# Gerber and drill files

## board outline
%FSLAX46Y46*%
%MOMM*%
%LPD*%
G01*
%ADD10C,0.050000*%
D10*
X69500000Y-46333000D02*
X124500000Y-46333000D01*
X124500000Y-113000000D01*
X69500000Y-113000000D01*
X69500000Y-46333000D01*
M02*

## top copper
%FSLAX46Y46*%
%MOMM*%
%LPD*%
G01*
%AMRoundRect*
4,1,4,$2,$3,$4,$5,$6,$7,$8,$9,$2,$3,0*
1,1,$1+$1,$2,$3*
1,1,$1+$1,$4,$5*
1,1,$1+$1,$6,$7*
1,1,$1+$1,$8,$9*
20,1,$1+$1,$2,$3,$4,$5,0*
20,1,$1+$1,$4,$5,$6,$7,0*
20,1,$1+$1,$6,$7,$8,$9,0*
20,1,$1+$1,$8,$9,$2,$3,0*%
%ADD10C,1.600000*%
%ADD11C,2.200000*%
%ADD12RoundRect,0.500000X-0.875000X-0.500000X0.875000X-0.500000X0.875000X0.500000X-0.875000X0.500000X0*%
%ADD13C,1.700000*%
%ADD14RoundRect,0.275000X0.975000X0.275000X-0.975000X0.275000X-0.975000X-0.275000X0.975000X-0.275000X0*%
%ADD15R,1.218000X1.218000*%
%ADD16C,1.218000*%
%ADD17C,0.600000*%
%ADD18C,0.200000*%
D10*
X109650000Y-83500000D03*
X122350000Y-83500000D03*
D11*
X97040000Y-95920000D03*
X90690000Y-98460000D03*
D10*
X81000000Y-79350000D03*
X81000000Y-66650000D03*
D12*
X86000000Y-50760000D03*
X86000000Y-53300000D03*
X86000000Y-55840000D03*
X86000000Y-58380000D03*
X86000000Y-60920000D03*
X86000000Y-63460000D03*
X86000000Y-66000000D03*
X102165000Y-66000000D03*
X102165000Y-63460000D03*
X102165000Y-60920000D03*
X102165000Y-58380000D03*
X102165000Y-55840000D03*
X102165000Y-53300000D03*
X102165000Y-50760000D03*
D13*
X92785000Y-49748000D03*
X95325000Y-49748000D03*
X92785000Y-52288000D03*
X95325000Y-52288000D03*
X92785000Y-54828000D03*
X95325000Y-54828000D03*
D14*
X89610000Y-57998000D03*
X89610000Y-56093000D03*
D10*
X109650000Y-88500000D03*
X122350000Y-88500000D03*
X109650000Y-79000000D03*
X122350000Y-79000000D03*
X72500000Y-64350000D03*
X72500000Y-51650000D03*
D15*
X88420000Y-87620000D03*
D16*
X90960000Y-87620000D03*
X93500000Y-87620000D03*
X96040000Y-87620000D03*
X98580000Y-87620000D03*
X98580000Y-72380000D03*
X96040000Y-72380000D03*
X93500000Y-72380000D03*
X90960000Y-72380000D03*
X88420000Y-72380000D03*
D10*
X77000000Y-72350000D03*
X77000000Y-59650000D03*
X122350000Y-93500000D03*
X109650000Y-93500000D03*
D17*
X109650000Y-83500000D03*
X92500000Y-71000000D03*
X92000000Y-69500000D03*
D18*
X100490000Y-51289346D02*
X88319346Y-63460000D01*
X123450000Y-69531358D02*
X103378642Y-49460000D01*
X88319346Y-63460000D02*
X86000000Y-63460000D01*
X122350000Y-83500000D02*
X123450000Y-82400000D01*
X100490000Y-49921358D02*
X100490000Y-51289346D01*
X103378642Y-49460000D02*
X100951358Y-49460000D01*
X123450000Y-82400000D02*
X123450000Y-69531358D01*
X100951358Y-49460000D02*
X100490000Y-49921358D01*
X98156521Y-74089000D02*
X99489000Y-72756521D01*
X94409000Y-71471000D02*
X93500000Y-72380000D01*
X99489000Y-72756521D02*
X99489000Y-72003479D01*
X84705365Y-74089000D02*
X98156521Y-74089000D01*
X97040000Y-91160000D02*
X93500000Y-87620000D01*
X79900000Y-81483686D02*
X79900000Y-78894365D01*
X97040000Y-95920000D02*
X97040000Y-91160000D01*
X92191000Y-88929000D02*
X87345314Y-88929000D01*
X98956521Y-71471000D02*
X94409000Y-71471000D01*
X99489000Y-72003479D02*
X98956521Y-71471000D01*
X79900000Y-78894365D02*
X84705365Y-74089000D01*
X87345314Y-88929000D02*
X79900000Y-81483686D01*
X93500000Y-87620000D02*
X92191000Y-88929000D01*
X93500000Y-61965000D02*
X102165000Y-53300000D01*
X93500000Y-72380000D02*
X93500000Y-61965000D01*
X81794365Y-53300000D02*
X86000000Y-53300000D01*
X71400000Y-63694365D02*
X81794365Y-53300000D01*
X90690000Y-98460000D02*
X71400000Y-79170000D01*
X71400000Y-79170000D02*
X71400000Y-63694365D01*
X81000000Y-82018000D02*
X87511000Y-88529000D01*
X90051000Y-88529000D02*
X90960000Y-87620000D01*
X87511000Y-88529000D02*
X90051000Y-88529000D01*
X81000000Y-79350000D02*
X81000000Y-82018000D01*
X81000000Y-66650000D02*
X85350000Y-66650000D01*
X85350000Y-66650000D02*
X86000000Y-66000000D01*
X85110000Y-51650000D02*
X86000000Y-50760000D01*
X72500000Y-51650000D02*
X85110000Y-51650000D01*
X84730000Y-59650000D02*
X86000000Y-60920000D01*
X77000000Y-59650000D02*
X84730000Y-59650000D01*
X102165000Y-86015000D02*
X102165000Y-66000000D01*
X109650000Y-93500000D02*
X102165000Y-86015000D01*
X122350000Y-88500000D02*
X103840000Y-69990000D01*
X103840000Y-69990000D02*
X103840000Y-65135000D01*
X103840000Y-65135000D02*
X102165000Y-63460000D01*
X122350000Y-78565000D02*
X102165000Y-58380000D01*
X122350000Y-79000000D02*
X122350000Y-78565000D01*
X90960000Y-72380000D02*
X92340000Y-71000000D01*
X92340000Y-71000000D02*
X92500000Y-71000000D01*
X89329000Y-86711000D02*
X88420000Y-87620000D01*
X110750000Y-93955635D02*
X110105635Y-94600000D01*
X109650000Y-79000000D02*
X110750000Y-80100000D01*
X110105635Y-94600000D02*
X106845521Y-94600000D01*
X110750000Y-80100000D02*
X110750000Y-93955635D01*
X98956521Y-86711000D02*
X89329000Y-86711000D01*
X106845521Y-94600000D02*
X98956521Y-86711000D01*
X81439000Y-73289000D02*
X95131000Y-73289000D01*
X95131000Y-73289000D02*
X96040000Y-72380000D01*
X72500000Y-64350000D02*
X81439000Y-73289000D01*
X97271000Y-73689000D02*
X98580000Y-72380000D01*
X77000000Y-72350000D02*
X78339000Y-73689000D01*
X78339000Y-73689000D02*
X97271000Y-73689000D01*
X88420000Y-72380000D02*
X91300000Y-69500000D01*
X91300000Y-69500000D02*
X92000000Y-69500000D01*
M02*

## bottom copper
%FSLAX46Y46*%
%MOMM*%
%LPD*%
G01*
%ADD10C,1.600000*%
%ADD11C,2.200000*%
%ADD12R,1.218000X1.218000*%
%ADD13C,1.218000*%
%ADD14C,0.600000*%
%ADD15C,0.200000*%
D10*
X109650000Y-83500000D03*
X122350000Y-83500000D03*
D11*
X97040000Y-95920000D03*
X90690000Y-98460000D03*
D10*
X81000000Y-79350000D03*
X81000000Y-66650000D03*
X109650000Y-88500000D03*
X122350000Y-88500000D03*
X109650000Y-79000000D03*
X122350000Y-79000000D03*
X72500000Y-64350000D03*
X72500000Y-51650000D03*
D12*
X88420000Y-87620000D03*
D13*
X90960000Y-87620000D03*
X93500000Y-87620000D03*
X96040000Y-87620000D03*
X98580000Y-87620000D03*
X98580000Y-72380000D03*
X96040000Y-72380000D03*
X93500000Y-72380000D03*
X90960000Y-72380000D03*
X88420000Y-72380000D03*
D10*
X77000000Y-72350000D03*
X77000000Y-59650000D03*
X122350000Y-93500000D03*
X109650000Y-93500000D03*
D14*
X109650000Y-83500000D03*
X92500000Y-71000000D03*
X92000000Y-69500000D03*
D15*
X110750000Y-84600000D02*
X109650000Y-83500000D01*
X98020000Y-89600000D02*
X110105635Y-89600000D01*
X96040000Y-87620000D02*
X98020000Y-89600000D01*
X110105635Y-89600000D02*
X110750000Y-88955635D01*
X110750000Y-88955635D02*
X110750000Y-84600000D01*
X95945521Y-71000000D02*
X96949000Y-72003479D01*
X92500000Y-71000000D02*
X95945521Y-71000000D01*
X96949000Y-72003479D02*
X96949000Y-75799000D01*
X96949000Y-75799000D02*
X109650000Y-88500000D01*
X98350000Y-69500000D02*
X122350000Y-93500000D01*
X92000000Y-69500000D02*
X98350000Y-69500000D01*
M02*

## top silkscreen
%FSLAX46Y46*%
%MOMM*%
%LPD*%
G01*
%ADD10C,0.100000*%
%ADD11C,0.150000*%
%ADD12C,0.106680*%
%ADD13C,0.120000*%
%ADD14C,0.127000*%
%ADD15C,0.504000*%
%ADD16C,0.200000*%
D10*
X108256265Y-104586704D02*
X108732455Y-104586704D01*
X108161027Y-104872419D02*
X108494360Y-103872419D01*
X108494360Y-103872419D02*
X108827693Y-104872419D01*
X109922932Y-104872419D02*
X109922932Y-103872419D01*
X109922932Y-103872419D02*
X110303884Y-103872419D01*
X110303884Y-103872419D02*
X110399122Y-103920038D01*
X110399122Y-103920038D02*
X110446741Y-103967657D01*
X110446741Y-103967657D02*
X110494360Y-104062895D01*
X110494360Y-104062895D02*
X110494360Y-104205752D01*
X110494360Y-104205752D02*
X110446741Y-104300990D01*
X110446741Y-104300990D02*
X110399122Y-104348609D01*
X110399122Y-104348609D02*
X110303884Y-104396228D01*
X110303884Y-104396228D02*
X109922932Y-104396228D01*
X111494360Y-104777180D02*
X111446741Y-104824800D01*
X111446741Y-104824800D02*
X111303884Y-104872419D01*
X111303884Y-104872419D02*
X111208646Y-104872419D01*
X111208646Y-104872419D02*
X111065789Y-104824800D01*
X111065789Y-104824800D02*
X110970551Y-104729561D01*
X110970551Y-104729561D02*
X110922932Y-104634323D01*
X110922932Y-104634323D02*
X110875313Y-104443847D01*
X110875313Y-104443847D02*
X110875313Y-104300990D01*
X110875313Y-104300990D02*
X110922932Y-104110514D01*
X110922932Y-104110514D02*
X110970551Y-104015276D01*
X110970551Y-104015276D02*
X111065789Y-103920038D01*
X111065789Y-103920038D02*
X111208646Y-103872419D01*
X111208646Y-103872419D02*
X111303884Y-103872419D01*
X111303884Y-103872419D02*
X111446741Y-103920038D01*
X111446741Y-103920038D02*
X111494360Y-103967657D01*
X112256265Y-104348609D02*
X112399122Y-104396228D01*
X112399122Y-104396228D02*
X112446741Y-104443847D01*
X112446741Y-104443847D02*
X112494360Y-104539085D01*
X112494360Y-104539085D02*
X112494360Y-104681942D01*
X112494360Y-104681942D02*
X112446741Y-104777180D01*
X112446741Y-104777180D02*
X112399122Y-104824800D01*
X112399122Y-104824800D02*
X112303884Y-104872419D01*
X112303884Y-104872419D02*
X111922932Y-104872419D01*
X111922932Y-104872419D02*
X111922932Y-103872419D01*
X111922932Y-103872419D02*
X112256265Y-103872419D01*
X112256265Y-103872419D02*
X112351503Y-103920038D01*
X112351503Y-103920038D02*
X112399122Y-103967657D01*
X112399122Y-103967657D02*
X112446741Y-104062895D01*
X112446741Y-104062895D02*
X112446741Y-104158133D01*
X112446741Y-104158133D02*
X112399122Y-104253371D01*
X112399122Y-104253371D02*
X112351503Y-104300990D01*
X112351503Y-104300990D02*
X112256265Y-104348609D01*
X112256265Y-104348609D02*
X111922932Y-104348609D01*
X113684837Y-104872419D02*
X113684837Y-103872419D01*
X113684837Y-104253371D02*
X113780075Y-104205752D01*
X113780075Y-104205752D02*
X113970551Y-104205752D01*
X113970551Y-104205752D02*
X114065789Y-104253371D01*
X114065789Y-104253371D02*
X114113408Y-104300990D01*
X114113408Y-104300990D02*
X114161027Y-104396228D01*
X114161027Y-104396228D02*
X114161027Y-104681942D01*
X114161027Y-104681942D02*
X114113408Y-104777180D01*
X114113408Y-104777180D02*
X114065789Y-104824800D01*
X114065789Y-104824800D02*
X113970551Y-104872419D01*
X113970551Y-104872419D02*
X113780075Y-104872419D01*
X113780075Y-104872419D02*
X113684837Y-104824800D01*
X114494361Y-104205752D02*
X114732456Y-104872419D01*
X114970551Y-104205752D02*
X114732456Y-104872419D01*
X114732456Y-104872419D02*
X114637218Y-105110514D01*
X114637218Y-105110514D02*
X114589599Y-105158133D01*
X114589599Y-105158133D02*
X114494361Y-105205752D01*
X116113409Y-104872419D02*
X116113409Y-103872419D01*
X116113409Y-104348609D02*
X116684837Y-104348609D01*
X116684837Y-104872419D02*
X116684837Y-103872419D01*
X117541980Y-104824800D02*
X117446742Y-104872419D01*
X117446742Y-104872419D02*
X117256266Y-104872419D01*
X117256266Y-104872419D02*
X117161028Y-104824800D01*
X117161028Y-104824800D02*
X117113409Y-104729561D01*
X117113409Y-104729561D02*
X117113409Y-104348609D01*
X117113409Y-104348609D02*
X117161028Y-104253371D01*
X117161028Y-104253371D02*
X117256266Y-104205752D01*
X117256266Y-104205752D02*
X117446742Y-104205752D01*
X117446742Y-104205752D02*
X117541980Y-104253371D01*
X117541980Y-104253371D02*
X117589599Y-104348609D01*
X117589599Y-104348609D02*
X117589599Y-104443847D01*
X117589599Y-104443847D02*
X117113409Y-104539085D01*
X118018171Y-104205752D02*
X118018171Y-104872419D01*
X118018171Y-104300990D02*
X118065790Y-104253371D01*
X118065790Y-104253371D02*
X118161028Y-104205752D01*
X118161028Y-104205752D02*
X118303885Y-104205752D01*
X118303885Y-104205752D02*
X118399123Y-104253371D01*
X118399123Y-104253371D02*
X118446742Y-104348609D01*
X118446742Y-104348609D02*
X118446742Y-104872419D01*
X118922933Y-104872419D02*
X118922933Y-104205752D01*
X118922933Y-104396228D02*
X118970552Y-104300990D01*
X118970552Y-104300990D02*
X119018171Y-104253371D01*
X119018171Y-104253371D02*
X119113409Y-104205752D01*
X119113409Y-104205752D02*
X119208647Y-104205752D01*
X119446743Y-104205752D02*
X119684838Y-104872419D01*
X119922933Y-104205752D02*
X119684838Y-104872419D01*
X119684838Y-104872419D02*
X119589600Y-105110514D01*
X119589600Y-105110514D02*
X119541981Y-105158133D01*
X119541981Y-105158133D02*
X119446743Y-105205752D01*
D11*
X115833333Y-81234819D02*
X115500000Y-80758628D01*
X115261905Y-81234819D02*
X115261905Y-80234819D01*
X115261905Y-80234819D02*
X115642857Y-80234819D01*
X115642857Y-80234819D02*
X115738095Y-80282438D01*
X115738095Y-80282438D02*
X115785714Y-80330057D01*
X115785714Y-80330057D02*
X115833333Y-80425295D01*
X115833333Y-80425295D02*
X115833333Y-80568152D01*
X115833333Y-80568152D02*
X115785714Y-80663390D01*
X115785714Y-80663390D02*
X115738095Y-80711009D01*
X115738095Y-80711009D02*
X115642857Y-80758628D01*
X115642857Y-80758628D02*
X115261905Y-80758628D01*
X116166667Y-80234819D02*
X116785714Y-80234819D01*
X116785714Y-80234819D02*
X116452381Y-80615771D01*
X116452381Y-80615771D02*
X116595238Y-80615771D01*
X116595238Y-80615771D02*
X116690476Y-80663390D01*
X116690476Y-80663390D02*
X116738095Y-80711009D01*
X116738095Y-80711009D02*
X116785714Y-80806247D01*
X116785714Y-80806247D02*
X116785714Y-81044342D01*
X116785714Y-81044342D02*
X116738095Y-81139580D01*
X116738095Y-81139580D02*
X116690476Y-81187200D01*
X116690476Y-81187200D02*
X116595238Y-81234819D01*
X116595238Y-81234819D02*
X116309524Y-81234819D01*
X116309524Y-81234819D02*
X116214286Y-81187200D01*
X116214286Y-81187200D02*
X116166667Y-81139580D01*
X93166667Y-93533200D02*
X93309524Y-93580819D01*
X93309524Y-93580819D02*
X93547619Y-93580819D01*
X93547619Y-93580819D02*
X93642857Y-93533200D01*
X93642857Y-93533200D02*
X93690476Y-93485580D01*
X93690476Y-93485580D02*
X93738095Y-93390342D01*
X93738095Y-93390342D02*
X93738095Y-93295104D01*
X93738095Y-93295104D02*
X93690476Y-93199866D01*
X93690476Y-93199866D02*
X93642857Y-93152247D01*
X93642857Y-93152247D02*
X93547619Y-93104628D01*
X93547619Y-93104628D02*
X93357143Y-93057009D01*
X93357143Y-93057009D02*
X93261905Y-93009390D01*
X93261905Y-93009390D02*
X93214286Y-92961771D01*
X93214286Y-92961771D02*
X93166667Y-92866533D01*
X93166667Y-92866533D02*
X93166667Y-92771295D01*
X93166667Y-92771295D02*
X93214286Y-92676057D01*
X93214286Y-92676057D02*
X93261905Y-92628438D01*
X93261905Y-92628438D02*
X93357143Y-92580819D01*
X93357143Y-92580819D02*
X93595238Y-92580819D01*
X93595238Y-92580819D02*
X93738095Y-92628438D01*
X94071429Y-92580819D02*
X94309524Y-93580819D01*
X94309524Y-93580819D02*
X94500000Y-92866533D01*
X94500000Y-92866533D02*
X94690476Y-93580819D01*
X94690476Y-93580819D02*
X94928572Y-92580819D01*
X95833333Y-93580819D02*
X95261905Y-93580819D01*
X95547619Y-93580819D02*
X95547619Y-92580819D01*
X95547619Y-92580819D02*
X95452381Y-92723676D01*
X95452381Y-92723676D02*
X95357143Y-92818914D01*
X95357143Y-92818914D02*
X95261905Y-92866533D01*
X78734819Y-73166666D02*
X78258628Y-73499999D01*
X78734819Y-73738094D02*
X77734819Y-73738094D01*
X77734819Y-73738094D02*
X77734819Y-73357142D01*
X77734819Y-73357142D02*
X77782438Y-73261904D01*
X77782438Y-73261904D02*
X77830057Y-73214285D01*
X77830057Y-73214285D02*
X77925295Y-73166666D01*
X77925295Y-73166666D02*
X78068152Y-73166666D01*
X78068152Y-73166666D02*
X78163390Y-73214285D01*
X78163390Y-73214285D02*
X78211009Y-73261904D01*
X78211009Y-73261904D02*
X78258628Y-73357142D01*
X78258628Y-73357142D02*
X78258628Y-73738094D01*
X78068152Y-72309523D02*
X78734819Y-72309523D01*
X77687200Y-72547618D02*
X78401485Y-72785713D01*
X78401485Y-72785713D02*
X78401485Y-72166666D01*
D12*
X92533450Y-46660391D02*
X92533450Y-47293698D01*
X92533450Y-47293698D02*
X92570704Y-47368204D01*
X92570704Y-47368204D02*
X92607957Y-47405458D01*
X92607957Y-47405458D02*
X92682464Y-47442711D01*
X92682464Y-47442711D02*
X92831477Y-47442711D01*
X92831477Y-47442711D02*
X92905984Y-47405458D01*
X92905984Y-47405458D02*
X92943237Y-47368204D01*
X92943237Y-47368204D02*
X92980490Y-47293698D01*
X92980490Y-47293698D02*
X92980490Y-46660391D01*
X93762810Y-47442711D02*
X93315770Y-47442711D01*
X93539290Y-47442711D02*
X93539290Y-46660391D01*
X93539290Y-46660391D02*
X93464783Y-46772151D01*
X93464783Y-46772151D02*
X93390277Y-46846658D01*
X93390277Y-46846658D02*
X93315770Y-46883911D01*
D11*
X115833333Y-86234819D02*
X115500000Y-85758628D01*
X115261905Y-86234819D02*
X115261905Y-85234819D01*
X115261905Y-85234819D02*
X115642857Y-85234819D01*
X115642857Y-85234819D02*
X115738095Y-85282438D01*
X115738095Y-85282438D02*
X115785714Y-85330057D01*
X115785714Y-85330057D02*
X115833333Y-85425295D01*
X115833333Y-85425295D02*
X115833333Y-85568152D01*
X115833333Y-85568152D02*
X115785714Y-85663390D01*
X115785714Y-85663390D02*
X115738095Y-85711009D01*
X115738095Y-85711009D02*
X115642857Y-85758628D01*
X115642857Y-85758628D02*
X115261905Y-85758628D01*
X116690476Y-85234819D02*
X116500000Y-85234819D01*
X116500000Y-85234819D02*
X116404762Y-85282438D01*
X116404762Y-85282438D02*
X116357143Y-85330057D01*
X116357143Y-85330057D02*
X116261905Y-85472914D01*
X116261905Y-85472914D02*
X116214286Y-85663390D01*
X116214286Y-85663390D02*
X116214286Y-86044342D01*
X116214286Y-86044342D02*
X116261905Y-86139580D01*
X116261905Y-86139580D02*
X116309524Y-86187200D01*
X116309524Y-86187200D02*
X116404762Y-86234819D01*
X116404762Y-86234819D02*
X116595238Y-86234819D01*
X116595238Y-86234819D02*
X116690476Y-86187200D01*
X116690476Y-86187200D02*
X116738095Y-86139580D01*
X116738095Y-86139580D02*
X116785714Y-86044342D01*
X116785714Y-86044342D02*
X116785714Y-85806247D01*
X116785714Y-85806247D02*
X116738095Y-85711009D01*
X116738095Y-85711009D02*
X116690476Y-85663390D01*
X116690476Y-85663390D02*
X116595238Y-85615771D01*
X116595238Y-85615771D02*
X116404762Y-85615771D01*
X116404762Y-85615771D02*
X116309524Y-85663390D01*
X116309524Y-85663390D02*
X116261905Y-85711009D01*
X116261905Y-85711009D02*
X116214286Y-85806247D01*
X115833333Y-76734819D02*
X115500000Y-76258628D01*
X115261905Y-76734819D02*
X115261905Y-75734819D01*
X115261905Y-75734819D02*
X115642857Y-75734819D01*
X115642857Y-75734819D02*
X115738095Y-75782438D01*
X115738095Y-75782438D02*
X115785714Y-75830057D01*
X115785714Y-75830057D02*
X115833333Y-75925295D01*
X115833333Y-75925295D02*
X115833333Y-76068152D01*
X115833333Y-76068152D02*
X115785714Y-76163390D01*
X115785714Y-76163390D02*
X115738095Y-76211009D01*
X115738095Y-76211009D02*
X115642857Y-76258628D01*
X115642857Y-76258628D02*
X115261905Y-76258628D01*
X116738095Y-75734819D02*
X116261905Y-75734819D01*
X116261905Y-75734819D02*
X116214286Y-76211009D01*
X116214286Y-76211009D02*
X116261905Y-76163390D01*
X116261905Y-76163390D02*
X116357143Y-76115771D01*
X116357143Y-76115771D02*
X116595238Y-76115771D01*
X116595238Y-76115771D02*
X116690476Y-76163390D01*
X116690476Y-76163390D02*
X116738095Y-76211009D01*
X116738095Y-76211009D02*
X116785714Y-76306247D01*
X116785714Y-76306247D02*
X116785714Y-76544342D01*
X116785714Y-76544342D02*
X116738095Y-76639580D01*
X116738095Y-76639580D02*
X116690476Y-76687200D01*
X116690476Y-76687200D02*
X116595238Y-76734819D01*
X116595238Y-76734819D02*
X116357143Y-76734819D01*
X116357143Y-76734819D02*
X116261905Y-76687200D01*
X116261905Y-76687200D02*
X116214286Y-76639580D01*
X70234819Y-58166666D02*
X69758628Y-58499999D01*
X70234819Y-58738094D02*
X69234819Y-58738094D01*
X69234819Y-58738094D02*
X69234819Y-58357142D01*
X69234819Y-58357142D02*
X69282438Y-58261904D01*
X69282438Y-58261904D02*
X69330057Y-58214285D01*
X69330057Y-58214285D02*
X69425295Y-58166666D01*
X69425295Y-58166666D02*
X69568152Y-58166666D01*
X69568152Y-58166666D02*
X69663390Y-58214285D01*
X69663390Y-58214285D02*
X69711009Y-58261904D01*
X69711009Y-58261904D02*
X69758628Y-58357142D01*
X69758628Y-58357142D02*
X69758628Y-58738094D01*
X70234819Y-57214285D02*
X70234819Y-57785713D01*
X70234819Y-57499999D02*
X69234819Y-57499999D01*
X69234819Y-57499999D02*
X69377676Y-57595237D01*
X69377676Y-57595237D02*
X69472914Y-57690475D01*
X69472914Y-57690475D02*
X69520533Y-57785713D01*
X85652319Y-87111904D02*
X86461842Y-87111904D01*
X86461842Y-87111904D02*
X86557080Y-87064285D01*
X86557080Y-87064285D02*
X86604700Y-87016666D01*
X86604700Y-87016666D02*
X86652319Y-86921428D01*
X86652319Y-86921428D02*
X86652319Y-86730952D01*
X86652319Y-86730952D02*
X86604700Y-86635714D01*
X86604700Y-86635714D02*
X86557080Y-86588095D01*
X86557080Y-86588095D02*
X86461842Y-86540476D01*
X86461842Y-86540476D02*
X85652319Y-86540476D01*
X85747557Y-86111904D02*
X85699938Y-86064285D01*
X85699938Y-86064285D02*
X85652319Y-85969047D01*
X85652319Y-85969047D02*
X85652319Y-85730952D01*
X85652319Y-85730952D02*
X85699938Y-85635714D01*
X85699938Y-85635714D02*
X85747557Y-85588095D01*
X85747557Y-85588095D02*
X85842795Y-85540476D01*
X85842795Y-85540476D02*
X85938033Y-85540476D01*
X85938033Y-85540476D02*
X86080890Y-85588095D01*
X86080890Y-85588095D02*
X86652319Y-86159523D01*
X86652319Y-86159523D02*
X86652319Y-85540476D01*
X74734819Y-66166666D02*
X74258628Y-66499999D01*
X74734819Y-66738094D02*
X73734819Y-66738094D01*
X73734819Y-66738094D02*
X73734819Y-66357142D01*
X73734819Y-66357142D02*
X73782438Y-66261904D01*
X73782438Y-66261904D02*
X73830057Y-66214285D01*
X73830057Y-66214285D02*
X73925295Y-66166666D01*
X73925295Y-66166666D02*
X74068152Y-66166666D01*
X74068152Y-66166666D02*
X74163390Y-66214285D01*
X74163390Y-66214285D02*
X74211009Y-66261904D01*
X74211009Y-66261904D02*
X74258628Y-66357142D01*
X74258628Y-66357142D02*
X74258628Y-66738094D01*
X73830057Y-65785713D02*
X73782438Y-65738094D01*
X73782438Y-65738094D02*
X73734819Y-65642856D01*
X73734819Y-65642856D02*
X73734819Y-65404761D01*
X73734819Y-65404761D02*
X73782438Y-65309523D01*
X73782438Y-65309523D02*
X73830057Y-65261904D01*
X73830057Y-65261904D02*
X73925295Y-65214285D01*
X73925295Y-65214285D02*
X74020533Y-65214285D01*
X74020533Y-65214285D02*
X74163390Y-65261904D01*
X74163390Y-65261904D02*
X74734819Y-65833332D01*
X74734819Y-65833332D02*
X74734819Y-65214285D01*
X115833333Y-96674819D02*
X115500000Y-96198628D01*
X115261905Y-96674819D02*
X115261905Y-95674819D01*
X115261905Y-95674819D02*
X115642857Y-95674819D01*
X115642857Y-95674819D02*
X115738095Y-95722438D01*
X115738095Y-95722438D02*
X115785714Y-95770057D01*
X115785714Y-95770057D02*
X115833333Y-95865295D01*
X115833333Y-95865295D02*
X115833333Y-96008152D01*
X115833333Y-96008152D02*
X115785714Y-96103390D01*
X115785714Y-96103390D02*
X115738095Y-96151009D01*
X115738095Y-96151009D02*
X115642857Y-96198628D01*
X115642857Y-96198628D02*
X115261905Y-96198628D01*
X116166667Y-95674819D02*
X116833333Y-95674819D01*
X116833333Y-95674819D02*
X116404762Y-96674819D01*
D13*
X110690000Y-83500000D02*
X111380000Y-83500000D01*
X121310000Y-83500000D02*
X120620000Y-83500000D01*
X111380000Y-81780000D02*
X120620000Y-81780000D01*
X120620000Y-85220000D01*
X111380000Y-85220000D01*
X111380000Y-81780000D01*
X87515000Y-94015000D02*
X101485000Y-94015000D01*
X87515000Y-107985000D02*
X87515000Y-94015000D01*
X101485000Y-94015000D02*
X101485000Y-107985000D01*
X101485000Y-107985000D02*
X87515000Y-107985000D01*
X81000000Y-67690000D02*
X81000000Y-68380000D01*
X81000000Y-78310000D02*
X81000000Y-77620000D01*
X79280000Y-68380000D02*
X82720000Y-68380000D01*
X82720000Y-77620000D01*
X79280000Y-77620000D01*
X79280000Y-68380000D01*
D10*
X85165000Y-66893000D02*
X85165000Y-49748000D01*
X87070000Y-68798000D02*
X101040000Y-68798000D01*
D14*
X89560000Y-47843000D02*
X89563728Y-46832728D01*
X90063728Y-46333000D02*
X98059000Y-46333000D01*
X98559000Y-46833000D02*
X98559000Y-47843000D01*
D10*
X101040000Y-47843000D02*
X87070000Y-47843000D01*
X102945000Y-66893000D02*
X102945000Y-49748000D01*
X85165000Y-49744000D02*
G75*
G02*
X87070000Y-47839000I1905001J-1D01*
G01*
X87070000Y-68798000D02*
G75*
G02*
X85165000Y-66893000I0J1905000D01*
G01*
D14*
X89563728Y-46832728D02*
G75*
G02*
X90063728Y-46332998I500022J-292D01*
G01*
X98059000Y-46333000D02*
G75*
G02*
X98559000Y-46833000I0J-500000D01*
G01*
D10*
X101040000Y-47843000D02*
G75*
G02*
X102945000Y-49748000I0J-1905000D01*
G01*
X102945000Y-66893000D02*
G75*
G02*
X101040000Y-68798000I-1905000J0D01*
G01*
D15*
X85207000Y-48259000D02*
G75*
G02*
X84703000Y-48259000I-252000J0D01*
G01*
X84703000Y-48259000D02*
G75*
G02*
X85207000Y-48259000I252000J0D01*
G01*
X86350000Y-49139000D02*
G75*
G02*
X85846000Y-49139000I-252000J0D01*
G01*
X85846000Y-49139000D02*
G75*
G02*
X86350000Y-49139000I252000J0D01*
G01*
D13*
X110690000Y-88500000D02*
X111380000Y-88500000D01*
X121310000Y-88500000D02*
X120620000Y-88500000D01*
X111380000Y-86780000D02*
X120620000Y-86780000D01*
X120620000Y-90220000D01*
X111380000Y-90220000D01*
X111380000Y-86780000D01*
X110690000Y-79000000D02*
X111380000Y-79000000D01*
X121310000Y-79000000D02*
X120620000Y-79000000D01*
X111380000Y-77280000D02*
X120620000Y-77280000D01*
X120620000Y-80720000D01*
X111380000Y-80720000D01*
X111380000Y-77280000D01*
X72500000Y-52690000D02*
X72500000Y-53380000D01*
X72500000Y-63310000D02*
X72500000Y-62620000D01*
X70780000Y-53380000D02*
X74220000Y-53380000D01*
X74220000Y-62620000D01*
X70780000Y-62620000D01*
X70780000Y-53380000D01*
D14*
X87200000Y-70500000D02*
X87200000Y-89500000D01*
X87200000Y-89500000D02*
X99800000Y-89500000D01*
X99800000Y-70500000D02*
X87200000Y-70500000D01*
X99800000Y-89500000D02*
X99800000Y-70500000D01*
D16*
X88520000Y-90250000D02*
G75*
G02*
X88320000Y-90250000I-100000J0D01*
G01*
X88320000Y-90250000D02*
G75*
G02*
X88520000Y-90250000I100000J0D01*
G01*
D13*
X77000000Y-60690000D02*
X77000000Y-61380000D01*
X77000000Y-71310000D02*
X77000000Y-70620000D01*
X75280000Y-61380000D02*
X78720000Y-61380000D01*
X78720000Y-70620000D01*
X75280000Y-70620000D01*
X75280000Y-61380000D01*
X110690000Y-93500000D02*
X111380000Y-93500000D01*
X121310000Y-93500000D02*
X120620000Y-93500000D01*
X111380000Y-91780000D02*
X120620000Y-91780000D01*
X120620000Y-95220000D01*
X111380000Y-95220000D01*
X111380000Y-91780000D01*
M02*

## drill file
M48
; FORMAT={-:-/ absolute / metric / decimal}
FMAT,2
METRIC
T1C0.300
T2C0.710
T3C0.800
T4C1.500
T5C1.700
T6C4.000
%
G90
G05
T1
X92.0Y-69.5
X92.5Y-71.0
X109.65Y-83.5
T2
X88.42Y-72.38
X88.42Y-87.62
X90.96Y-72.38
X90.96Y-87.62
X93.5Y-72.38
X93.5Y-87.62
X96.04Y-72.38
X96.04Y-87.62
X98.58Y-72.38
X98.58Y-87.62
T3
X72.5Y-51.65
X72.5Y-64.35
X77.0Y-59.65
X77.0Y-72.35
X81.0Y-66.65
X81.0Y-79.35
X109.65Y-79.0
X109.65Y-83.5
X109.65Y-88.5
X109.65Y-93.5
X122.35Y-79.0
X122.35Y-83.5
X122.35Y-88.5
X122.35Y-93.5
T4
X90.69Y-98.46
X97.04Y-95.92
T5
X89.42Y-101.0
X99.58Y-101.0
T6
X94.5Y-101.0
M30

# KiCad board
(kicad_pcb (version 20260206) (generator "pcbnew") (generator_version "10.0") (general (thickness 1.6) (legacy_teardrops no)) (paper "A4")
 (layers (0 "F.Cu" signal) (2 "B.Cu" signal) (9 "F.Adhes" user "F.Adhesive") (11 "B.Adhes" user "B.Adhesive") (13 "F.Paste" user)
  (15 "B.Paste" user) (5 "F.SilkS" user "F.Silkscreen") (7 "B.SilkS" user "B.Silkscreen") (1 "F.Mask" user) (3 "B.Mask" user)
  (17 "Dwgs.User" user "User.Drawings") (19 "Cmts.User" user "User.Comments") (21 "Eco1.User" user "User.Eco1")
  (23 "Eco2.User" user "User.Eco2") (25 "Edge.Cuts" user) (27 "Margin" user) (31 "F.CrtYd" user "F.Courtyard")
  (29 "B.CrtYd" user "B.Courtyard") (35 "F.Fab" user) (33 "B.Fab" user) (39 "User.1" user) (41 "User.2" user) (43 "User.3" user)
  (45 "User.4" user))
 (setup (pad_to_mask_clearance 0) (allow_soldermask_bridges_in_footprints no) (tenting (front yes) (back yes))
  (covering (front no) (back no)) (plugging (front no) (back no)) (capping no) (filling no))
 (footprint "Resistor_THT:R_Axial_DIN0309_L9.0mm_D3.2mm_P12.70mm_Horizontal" (layer "F.Cu") (at 109.65 83.5)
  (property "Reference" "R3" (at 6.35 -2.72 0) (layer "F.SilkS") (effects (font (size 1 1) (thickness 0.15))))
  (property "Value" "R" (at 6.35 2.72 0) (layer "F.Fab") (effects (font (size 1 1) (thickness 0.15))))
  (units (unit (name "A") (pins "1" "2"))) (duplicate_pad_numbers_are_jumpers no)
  (fp_line (start 1.04 0) (end 1.73 0) (stroke (width 0.12) (type solid)) (layer "F.SilkS"))
  (fp_line (start 11.66 0) (end 10.97 0) (stroke (width 0.12) (type solid)) (layer "F.SilkS"))
  (fp_rect (start 1.73 -1.72) (end 10.97 1.72) (stroke (width 0.12) (type solid)) (fill no) (layer "F.SilkS"))
  (pad "1" thru_hole circle (at 0 0) (size 1.6 1.6) (drill 0.8) (layers "*.Cu" "*.Mask") (remove_unused_layers no) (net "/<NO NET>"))
  (pad "2" thru_hole circle (at 12.7 0) (size 1.6 1.6) (drill 0.8) (layers "*.Cu" "*.Mask") (remove_unused_layers no) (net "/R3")))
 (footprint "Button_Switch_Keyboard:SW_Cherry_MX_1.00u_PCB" (layer "F.Cu") (at 97.04 95.92)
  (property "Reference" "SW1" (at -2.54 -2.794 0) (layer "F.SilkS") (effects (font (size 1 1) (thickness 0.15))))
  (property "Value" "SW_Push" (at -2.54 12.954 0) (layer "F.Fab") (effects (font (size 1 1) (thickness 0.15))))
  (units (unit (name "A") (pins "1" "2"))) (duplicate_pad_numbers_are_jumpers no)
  (fp_line (start -9.525 -1.905) (end 4.445 -1.905) (stroke (width 0.12) (type solid)) (layer "F.SilkS"))
  (fp_line (start -9.525 12.065) (end -9.525 -1.905) (stroke (width 0.12) (type solid)) (layer "F.SilkS"))
  (fp_line (start 4.445 -1.905) (end 4.445 12.065) (stroke (width 0.12) (type solid)) (layer "F.SilkS"))
  (fp_line (start 4.445 12.065) (end -9.525 12.065) (stroke (width 0.12) (type solid)) (layer "F.SilkS"))
  (pad "" np_thru_hole circle (at -7.62 5.08) (size 1.7 1.7) (drill 1.7) (layers "*.Cu" "*.Mask"))
  (pad "" np_thru_hole circle (at -2.54 5.08) (size 4 4) (drill 4) (layers "*.Cu" "*.Mask"))
  (pad "" np_thru_hole circle (at 2.54 5.08) (size 1.7 1.7) (drill 1.7) (layers "*.Cu" "*.Mask"))
  (pad "1" thru_hole circle (at 0 0) (size 2.2 2.2) (drill 1.5) (layers "*.Cu" "*.Mask") (remove_unused_layers no) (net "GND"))
  (pad "2" thru_hole circle (at -6.35 2.54) (size 2.2 2.2) (drill 1.5) (layers "*.Cu" "*.Mask") (remove_unused_layers no) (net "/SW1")))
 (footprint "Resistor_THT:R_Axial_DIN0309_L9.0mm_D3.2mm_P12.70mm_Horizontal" (layer "F.Cu") (at 81 79.35 90)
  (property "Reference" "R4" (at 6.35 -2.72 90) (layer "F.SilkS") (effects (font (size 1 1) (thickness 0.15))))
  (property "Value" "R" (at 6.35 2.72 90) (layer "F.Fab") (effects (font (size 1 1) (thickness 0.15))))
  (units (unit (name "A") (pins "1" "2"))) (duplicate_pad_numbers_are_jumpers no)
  (fp_line (start 11.66 0) (end 10.97 0) (stroke (width 0.12) (type solid)) (layer "F.SilkS"))
  (fp_line (start 1.04 0) (end 1.73 0) (stroke (width 0.12) (type solid)) (layer "F.SilkS"))
  (fp_rect (start 1.73 -1.72) (end 10.97 1.72) (stroke (width 0.12) (type solid)) (fill no) (layer "F.SilkS"))
  (pad "1" thru_hole circle (at 0 0 90) (size 1.6 1.6) (drill 0.8) (layers "*.Cu" "*.Mask") (remove_unused_layers no) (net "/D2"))
  (pad "2" thru_hole circle (at 12.7 0 90) (size 1.6 1.6) (drill 0.8) (layers "*.Cu" "*.Mask") (remove_unused_layers no) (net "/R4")))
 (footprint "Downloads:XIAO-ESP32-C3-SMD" (layer "F.Cu") (at 85.165 68.88)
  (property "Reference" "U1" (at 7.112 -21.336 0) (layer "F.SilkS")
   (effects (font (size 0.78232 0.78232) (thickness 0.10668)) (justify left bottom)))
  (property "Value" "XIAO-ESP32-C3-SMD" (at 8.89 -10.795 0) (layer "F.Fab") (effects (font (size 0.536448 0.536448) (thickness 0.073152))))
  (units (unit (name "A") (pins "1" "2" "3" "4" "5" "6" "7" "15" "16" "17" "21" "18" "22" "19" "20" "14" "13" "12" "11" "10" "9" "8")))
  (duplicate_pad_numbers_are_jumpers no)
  (fp_line (start 0 -1.987) (end 0 -19.132) (stroke (width 0.1) (type solid)) (layer "F.SilkS"))
  (fp_line (start 1.905 -0.082) (end 15.875 -0.082) (stroke (width 0.1) (type solid)) (layer "F.SilkS"))
  (fp_line (start 4.395 -21.037) (end 4.398728 -22.047272) (stroke (width 0.127) (type solid)) (layer "F.SilkS"))
  (fp_line (start 4.898728 -22.547) (end 12.894 -22.547) (stroke (width 0.127) (type solid)) (layer "F.SilkS"))
  (fp_line (start 13.394 -22.047) (end 13.394 -21.037) (stroke (width 0.127) (type solid)) (layer "F.SilkS"))
  (fp_line (start 15.875 -21.037) (end 1.905 -21.037) (stroke (width 0.1) (type solid)) (layer "F.SilkS"))
  (fp_line (start 17.78 -1.987) (end 17.78 -19.132) (stroke (width 0.1) (type solid)) (layer "F.SilkS"))
  (fp_arc (start 0 -19.136) (mid 0.557962 -20.483038) (end 1.905 -21.041) (stroke (width 0.1) (type solid)) (layer "F.SilkS"))
  (fp_arc (start 1.905 -0.082) (mid 0.557962 -0.639962) (end 0 -1.987) (stroke (width 0.1) (type solid)) (layer "F.SilkS"))
  (fp_arc (start 4.398728 -22.047272) (mid 4.545272 -22.40064) (end 4.898728 -22.547) (stroke (width 0.127) (type default))
   (layer "F.SilkS"))
  (fp_arc (start 12.894 -22.547) (mid 13.247553 -22.400553) (end 13.394 -22.047) (stroke (width 0.127) (type default)) (layer "F.SilkS"))
  (fp_arc (start 15.875 -21.037) (mid 17.222038 -20.479038) (end 17.78 -19.132) (stroke (width 0.1) (type solid)) (layer "F.SilkS"))
  (fp_arc (start 17.78 -1.987) (mid 17.222038 -0.639962) (end 15.875 -0.082) (stroke (width 0.1) (type solid)) (layer "F.SilkS"))
  (fp_circle (center -0.21 -20.621) (end -0.21 -20.875) (stroke (width 0.5) (type solid)) (fill yes) (layer "F.SilkS"))
  (fp_circle (center 0.933 -19.741) (end 0.933 -19.995) (stroke (width 0.5) (type solid)) (fill yes) (layer "F.SilkS"))
  (pad "1" smd roundrect (at 0.835 -18.12) (size 2.75 2) (layers "F.Cu" "F.Mask" "F.Paste") (roundrect_rratio 0.25) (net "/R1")
   (solder_mask_margin 0.0508) (thermal_bridge_angle 45))
  (pad "2" smd roundrect (at 0.835 -15.58) (size 2.75 2) (layers "F.Cu" "F.Mask" "F.Paste") (roundrect_rratio 0.25) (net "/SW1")
   (solder_mask_margin 0.0508) (thermal_bridge_angle 45))
  (pad "3" smd roundrect (at 0.835 -13.04) (size 2.75 2) (layers "F.Cu" "F.Mask" "F.Paste") (roundrect_rratio 0.25)
   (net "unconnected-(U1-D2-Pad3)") (solder_mask_margin 0.0508) (thermal_bridge_angle 45))
  (pad "4" smd roundrect (at 0.835 -10.5) (size 2.75 2) (layers "F.Cu" "F.Mask" "F.Paste") (roundrect_rratio 0.25)
   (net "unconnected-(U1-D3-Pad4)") (solder_mask_margin 0.0508) (thermal_bridge_angle 45))
  (pad "5" smd roundrect (at 0.835 -7.96) (size 2.75 2) (layers "F.Cu" "F.Mask" "F.Paste") (roundrect_rratio 0.25) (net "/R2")
   (solder_mask_margin 0.0508) (thermal_bridge_angle 45))
  (pad "6" smd roundrect (at 0.835 -5.42) (size 2.75 2) (layers "F.Cu" "F.Mask" "F.Paste") (roundrect_rratio 0.25) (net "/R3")
   (solder_mask_margin 0.0508) (thermal_bridge_angle 45))
  (pad "7" smd roundrect (at 0.835 -2.88) (size 2.75 2) (layers "F.Cu" "F.Mask" "F.Paste") (roundrect_rratio 0.25) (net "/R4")
   (solder_mask_margin 0.0508) (thermal_bridge_angle 45))
  (pad "8" smd roundrect (at 17 -2.88) (size 2.75 2) (layers "F.Cu" "F.Mask" "F.Paste") (roundrect_rratio 0.25) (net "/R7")
   (solder_mask_margin 0.0508) (thermal_bridge_angle 45))
  (pad "9" smd roundrect (at 17 -5.42) (size 2.75 2) (layers "F.Cu" "F.Mask" "F.Paste") (roundrect_rratio 0.25) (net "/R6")
   (solder_mask_margin 0.0508) (thermal_bridge_angle 45))
  (pad "10" smd roundrect (at 17 -7.96) (size 2.75 2) (layers "F.Cu" "F.Mask" "F.Paste") (roundrect_rratio 0.25)
   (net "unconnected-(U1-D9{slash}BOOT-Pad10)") (solder_mask_margin 0.0508) (thermal_bridge_angle 45))
  (pad "11" smd roundrect (at 17 -10.5) (size 2.75 2) (layers "F.Cu" "F.Mask" "F.Paste") (roundrect_rratio 0.25) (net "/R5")
   (solder_mask_margin 0.0508) (thermal_bridge_angle 45))
  (pad "12" smd roundrect (at 17 -13.04) (size 2.75 2) (layers "F.Cu" "F.Mask" "F.Paste") (roundrect_rratio 0.25) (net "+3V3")
   (solder_mask_margin 0.0508) (thermal_bridge_angle 45))
  (pad "13" smd roundrect (at 17 -15.58) (size 2.75 2) (layers "F.Cu" "F.Mask" "F.Paste") (roundrect_rratio 0.25) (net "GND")
   (solder_mask_margin 0.0508) (thermal_bridge_angle 45))
  (pad "14" smd roundrect (at 17 -18.12) (size 2.75 2) (layers "F.Cu" "F.Mask" "F.Paste") (roundrect_rratio 0.25) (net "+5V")
   (solder_mask_margin 0.0508) (thermal_bridge_angle 45))
  (pad "15" smd circle (at 7.62 -19.132) (size 1.7 1.7) (layers "F.Cu" "F.Mask" "F.Paste") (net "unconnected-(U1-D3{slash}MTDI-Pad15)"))
  (pad "16" smd circle (at 10.16 -19.132) (size 1.7 1.7) (layers "F.Cu" "F.Mask" "F.Paste") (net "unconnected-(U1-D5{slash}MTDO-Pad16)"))
  (pad "17" smd circle (at 7.62 -16.592) (size 1.7 1.7) (layers "F.Cu" "F.Mask" "F.Paste") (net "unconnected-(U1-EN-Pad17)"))
  (pad "18" smd circle (at 10.16 -16.592) (size 1.7 1.7) (layers "F.Cu" "F.Mask" "F.Paste") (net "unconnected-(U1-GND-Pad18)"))
  (pad "19" smd circle (at 7.62 -14.052) (size 1.7 1.7) (layers "F.Cu" "F.Mask" "F.Paste") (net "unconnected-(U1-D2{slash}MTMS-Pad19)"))
  (pad "20" smd circle (at 10.16 -14.052) (size 1.7 1.7) (layers "F.Cu" "F.Mask" "F.Paste") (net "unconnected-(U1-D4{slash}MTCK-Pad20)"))
  (pad "21" smd roundrect (at 4.445 -10.882 180) (size 2.5 1.1) (layers "F.Cu" "F.Mask" "F.Paste") (roundrect_rratio 0.25)
   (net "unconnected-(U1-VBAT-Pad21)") (thermal_bridge_angle 45))
  (pad "22" smd roundrect (at 4.445 -12.787 180) (size 2.5 1.1) (layers "F.Cu" "F.Mask" "F.Paste") (roundrect_rratio 0.25)
   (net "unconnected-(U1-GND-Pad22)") (thermal_bridge_angle 45)))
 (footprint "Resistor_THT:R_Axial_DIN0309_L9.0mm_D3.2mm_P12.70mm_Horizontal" (layer "F.Cu") (at 109.65 88.5)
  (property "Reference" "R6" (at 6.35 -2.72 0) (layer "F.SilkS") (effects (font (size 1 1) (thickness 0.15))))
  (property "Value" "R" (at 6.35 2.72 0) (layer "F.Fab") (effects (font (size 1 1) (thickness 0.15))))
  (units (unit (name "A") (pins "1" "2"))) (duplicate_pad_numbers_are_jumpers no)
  (fp_line (start 1.04 0) (end 1.73 0) (stroke (width 0.12) (type solid)) (layer "F.SilkS"))
  (fp_line (start 11.66 0) (end 10.97 0) (stroke (width 0.12) (type solid)) (layer "F.SilkS"))
  (fp_rect (start 1.73 -1.72) (end 10.97 1.72) (stroke (width 0.12) (type solid)) (fill no) (layer "F.SilkS"))
  (pad "1" thru_hole circle (at 0 0) (size 1.6 1.6) (drill 0.8) (layers "*.Cu" "*.Mask") (remove_unused_layers no) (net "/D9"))
  (pad "2" thru_hole circle (at 12.7 0) (size 1.6 1.6) (drill 0.8) (layers "*.Cu" "*.Mask") (remove_unused_layers no) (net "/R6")))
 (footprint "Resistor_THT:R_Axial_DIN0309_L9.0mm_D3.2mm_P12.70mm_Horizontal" (layer "F.Cu") (at 109.65 79)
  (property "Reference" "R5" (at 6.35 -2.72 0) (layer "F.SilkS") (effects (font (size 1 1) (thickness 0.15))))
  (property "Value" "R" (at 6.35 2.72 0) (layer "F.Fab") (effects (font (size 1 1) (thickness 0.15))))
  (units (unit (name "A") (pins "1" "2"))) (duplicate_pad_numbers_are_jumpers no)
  (fp_line (start 1.04 0) (end 1.73 0) (stroke (width 0.12) (type solid)) (layer "F.SilkS"))
  (fp_line (start 11.66 0) (end 10.97 0) (stroke (width 0.12) (type solid)) (layer "F.SilkS"))
  (fp_rect (start 1.73 -1.72) (end 10.97 1.72) (stroke (width 0.12) (type solid)) (fill no) (layer "F.SilkS"))
  (pad "1" thru_hole circle (at 0 0) (size 1.6 1.6) (drill 0.8) (layers "*.Cu" "*.Mask") (remove_unused_layers no) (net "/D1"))
  (pad "2" thru_hole circle (at 12.7 0) (size 1.6 1.6) (drill 0.8) (layers "*.Cu" "*.Mask") (remove_unused_layers no) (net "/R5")))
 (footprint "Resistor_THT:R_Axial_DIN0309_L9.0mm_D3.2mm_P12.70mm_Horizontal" (layer "F.Cu") (at 72.5 64.35 90)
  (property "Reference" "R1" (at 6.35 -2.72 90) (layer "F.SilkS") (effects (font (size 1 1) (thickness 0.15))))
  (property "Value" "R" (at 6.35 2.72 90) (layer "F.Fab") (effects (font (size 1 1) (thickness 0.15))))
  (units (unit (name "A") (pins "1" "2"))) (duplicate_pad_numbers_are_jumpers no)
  (fp_line (start 11.66 0) (end 10.97 0) (stroke (width 0.12) (type solid)) (layer "F.SilkS"))
  (fp_line (start 1.04 0) (end 1.73 0) (stroke (width 0.12) (type solid)) (layer "F.SilkS"))
  (fp_rect (start 1.73 -1.72) (end 10.97 1.72) (stroke (width 0.12) (type solid)) (fill no) (layer "F.SilkS"))
  (pad "1" thru_hole circle (at 0 0 90) (size 1.6 1.6) (drill 0.8) (layers "*.Cu" "*.Mask") (remove_unused_layers no) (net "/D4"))
  (pad "2" thru_hole circle (at 12.7 0 90) (size 1.6 1.6) (drill 0.8) (layers "*.Cu" "*.Mask") (remove_unused_layers no) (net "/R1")))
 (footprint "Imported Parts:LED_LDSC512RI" (layer "F.Cu") (at 93.5 80 90)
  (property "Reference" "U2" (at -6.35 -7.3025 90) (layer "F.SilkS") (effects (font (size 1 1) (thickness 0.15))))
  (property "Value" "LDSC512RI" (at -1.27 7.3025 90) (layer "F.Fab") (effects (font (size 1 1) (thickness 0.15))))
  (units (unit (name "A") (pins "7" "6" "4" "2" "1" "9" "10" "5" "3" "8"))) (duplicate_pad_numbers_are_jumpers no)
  (fp_line (start 9.5 -6.3) (end -9.5 -6.3) (stroke (width 0.127) (type solid)) (layer "F.SilkS"))
  (fp_line (start -9.5 -6.3) (end -9.5 6.3) (stroke (width 0.127) (type solid)) (layer "F.SilkS"))
  (fp_line (start 9.5 6.3) (end 9.5 -6.3) (stroke (width 0.127) (type solid)) (layer "F.SilkS"))
  (fp_line (start -9.5 6.3) (end 9.5 6.3) (stroke (width 0.127) (type solid)) (layer "F.SilkS"))
  (fp_circle (center -10.25 -5.08) (end -10.15 -5.08) (stroke (width 0.2) (type solid)) (fill no) (layer "F.SilkS"))
  (pad "1" thru_hole rect (at -7.62 -5.08 90) (size 1.218 1.218) (drill 0.71) (layers "*.Cu" "*.Mask") (remove_unused_layers no) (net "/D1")
   (solder_mask_margin 0.102))
  (pad "2" thru_hole circle (at -7.62 -2.54 90) (size 1.218 1.218) (drill 0.71) (layers "*.Cu" "*.Mask") (remove_unused_layers no)
   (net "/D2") (solder_mask_margin 0.102))
  (pad "3" thru_hole circle (at -7.62 0 90) (size 1.218 1.218) (drill 0.71) (layers "*.Cu" "*.Mask") (remove_unused_layers no) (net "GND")
   (solder_mask_margin 0.102))
  (pad "4" thru_hole circle (at -7.62 2.54 90) (size 1.218 1.218) (drill 0.71) (layers "*.Cu" "*.Mask") (remove_unused_layers no)
   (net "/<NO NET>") (solder_mask_margin 0.102))
  (pad "5" thru_hole circle (at -7.62 5.08 90) (size 1.218 1.218) (drill 0.71) (layers "*.Cu" "*.Mask") (remove_unused_layers no)
   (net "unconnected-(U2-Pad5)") (solder_mask_margin 0.102))
  (pad "6" thru_hole circle (at 7.62 5.08 90) (size 1.218 1.218) (drill 0.71) (layers "*.Cu" "*.Mask") (remove_unused_layers no) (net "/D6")
   (solder_mask_margin 0.102))
  (pad "7" thru_hole circle (at 7.62 2.54 90) (size 1.218 1.218) (drill 0.71) (layers "*.Cu" "*.Mask") (remove_unused_layers no) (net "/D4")
   (solder_mask_margin 0.102))
  (pad "8" thru_hole circle (at 7.62 0 90) (size 1.218 1.218) (drill 0.71) (layers "*.Cu" "*.Mask") (remove_unused_layers no) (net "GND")
   (solder_mask_margin 0.102))
  (pad "9" thru_hole circle (at 7.62 -2.54 90) (size 1.218 1.218) (drill 0.71) (layers "*.Cu" "*.Mask") (remove_unused_layers no)
   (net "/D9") (solder_mask_margin 0.102))
  (pad "10" thru_hole circle (at 7.62 -5.08 90) (size 1.218 1.218) (drill 0.71) (layers "*.Cu" "*.Mask") (remove_unused_layers no)
   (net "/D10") (solder_mask_margin 0.102)))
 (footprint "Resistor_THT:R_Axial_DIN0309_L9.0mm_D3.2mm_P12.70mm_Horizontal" (layer "F.Cu") (at 77 72.35 90)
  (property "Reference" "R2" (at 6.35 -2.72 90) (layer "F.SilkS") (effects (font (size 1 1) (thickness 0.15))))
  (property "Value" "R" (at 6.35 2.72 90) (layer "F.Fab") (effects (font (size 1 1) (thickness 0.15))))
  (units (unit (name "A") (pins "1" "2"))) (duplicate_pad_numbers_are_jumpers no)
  (fp_line (start 11.66 0) (end 10.97 0) (stroke (width 0.12) (type solid)) (layer "F.SilkS"))
  (fp_line (start 1.04 0) (end 1.73 0) (stroke (width 0.12) (type solid)) (layer "F.SilkS"))
  (fp_rect (start 1.73 -1.72) (end 10.97 1.72) (stroke (width 0.12) (type solid)) (fill no) (layer "F.SilkS"))
  (pad "1" thru_hole circle (at 0 0 90) (size 1.6 1.6) (drill 0.8) (layers "*.Cu" "*.Mask") (remove_unused_layers no) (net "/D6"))
  (pad "2" thru_hole circle (at 12.7 0 90) (size 1.6 1.6) (drill 0.8) (layers "*.Cu" "*.Mask") (remove_unused_layers no) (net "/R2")))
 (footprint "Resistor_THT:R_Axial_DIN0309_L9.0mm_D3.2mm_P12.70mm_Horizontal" (layer "F.Cu") (at 122.35 93.5 180)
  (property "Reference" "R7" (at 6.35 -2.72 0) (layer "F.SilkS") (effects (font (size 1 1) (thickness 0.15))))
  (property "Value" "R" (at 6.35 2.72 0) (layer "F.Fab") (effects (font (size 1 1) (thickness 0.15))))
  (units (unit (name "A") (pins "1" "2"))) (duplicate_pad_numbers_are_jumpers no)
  (fp_line (start 11.66 0) (end 10.97 0) (stroke (width 0.12) (type solid)) (layer "F.SilkS"))
  (fp_line (start 1.04 0) (end 1.73 0) (stroke (width 0.12) (type solid)) (layer "F.SilkS"))
  (fp_rect (start 1.73 -1.72) (end 10.97 1.72) (stroke (width 0.12) (type solid)) (fill no) (layer "F.SilkS"))
  (pad "1" thru_hole circle (at 0 0 180) (size 1.6 1.6) (drill 0.8) (layers "*.Cu" "*.Mask") (remove_unused_layers no) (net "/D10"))
  (pad "2" thru_hole circle (at 12.7 0 180) (size 1.6 1.6) (drill 0.8) (layers "*.Cu" "*.Mask") (remove_unused_layers no) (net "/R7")))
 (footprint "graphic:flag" (layer "B.Cu") (at 94.5 101 180)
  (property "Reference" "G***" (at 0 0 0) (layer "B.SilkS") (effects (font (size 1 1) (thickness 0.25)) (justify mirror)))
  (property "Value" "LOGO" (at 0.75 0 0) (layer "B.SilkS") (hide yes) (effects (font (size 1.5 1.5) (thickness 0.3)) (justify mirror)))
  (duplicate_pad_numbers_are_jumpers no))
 (gr_rect (start 69.5 46.333) (end 124.5 113) (stroke (width 0.05) (type default)) (fill no) (layer "Edge.Cuts"))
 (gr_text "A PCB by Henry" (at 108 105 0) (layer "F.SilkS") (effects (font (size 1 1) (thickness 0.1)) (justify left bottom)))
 (via (at 109.65 83.5) (size 0.6) (drill 0.3) (layers "F.Cu" "B.Cu") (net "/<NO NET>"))
 (segment (start 110.75 84.6) (end 109.65 83.5) (width 0.2) (layer "B.Cu") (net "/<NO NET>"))
 (segment (start 98.02 89.6) (end 110.105635 89.6) (width 0.2) (layer "B.Cu") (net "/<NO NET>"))
 (segment (start 96.04 87.62) (end 98.02 89.6) (width 0.2) (layer "B.Cu") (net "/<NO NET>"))
 (segment (start 110.105635 89.6) (end 110.75 88.955635) (width 0.2) (layer "B.Cu") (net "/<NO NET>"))
 (segment (start 110.75 88.955635) (end 110.75 84.6) (width 0.2) (layer "B.Cu") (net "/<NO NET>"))
 (segment (start 100.49 51.289346) (end 88.319346 63.46) (width 0.2) (layer "F.Cu") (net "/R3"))
 (segment (start 123.45 69.531358) (end 103.378642 49.46) (width 0.2) (layer "F.Cu") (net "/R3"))
 (segment (start 88.319346 63.46) (end 86 63.46) (width 0.2) (layer "F.Cu") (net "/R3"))
 (segment (start 122.35 83.5) (end 123.45 82.4) (width 0.2) (layer "F.Cu") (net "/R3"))
 (segment (start 100.49 49.921358) (end 100.49 51.289346) (width 0.2) (layer "F.Cu") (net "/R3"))
 (segment (start 103.378642 49.46) (end 100.951358 49.46) (width 0.2) (layer "F.Cu") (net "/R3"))
 (segment (start 123.45 82.4) (end 123.45 69.531358) (width 0.2) (layer "F.Cu") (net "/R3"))
 (segment (start 100.951358 49.46) (end 100.49 49.921358) (width 0.2) (layer "F.Cu") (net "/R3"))
 (segment (start 98.156521 74.089) (end 99.489 72.756521) (width 0.2) (layer "F.Cu") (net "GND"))
 (segment (start 94.409 71.471) (end 93.5 72.38) (width 0.2) (layer "F.Cu") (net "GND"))
 (segment (start 99.489 72.756521) (end 99.489 72.003479) (width 0.2) (layer "F.Cu") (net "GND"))
 (segment (start 84.705365 74.089) (end 98.156521 74.089) (width 0.2) (layer "F.Cu") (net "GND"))
 (segment (start 97.04 91.16) (end 93.5 87.62) (width 0.2) (layer "F.Cu") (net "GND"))
 (segment (start 79.9 81.483686) (end 79.9 78.894365) (width 0.2) (layer "F.Cu") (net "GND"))
 (segment (start 97.04 95.92) (end 97.04 91.16) (width 0.2) (layer "F.Cu") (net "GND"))
 (segment (start 92.191 88.929) (end 87.345314 88.929) (width 0.2) (layer "F.Cu") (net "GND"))
 (segment (start 98.956521 71.471) (end 94.409 71.471) (width 0.2) (layer "F.Cu") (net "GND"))
 (segment (start 99.489 72.003479) (end 98.956521 71.471) (width 0.2) (layer "F.Cu") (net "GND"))
 (segment (start 79.9 78.894365) (end 84.705365 74.089) (width 0.2) (layer "F.Cu") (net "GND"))
 (segment (start 87.345314 88.929) (end 79.9 81.483686) (width 0.2) (layer "F.Cu") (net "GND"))
 (segment (start 93.5 87.62) (end 92.191 88.929) (width 0.2) (layer "F.Cu") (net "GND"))
 (segment (start 93.5 61.965) (end 102.165 53.3) (width 0.2) (layer "F.Cu") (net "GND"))
 (segment (start 93.5 72.38) (end 93.5 61.965) (width 0.2) (layer "F.Cu") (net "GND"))
 (segment (start 81.794365 53.3) (end 86 53.3) (width 0.2) (layer "F.Cu") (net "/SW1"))
 (segment (start 71.4 63.694365) (end 81.794365 53.3) (width 0.2) (layer "F.Cu") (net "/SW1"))
 (segment (start 90.69 98.46) (end 71.4 79.17) (width 0.2) (layer "F.Cu") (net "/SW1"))
 (segment (start 71.4 79.17) (end 71.4 63.694365) (width 0.2) (layer "F.Cu") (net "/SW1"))
 (segment (start 81 82.018) (end 87.511 88.529) (width 0.2) (layer "F.Cu") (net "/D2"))
 (segment (start 90.051 88.529) (end 90.96 87.62) (width 0.2) (layer "F.Cu") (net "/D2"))
 (segment (start 87.511 88.529) (end 90.051 88.529) (width 0.2) (layer "F.Cu") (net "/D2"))
 (segment (start 81 79.35) (end 81 82.018) (width 0.2) (layer "F.Cu") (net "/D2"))
 (segment (start 81 66.65) (end 85.35 66.65) (width 0.2) (layer "F.Cu") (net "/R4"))
 (segment (start 85.35 66.65) (end 86 66) (width 0.2) (layer "F.Cu") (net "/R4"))
 (segment (start 85.11 51.65) (end 86 50.76) (width 0.2) (layer "F.Cu") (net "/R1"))
 (segment (start 72.5 51.65) (end 85.11 51.65) (width 0.2) (layer "F.Cu") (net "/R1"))
 (segment (start 84.73 59.65) (end 86 60.92) (width 0.2) (layer "F.Cu") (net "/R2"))
 (segment (start 77 59.65) (end 84.73 59.65) (width 0.2) (layer "F.Cu") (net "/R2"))
 (segment (start 102.165 86.015) (end 102.165 66) (width 0.2) (layer "F.Cu") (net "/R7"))
 (segment (start 109.65 93.5) (end 102.165 86.015) (width 0.2) (layer "F.Cu") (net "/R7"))
 (segment (start 122.35 88.5) (end 103.84 69.99) (width 0.2) (layer "F.Cu") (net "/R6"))
 (segment (start 103.84 69.99) (end 103.84 65.135) (width 0.2) (layer "F.Cu") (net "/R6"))
 (segment (start 103.84 65.135) (end 102.165 63.46) (width 0.2) (layer "F.Cu") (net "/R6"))
 (segment (start 122.35 78.565) (end 102.165 58.38) (width 0.2) (layer "F.Cu") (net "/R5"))
 (segment (start 122.35 79) (end 122.35 78.565) (width 0.2) (layer "F.Cu") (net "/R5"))
 (segment (start 90.96 72.38) (end 92.34 71) (width 0.2) (layer "F.Cu") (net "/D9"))
 (segment (start 92.34 71) (end 92.5 71) (width 0.2) (layer "F.Cu") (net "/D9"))
 (via (at 92.5 71) (size 0.6) (drill 0.3) (layers "F.Cu" "B.Cu") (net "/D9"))
 (segment (start 95.945521 71) (end 96.949 72.003479) (width 0.2) (layer "B.Cu") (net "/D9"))
 (segment (start 92.5 71) (end 95.945521 71) (width 0.2) (layer "B.Cu") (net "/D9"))
 (segment (start 96.949 72.003479) (end 96.949 75.799) (width 0.2) (layer "B.Cu") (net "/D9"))
 (segment (start 96.949 75.799) (end 109.65 88.5) (width 0.2) (layer "B.Cu") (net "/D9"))
 (segment (start 89.329 86.711) (end 88.42 87.62) (width 0.2) (layer "F.Cu") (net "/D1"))
 (segment (start 110.75 93.955635) (end 110.105635 94.6) (width 0.2) (layer "F.Cu") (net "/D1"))
 (segment (start 109.65 79) (end 110.75 80.1) (width 0.2) (layer "F.Cu") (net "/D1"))
 (segment (start 110.105635 94.6) (end 106.845521 94.6) (width 0.2) (layer "F.Cu") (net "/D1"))
 (segment (start 110.75 80.1) (end 110.75 93.955635) (width 0.2) (layer "F.Cu") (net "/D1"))
 (segment (start 98.956521 86.711) (end 89.329 86.711) (width 0.2) (layer "F.Cu") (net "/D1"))
 (segment (start 106.845521 94.6) (end 98.956521 86.711) (width 0.2) (layer "F.Cu") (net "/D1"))
 (segment (start 81.439 73.289) (end 95.131 73.289) (width 0.2) (layer "F.Cu") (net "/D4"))
 (segment (start 95.131 73.289) (end 96.04 72.38) (width 0.2) (layer "F.Cu") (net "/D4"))
 (segment (start 72.5 64.35) (end 81.439 73.289) (width 0.2) (layer "F.Cu") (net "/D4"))
 (segment (start 97.271 73.689) (end 98.58 72.38) (width 0.2) (layer "F.Cu") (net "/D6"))
 (segment (start 77 72.35) (end 78.339 73.689) (width 0.2) (layer "F.Cu") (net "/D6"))
 (segment (start 78.339 73.689) (end 97.271 73.689) (width 0.2) (layer "F.Cu") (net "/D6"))
 (segment (start 88.42 72.38) (end 91.3 69.5) (width 0.2) (layer "F.Cu") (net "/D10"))
 (segment (start 91.3 69.5) (end 92 69.5) (width 0.2) (layer "F.Cu") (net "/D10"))
 (via (at 92 69.5) (size 0.6) (drill 0.3) (layers "F.Cu" "B.Cu") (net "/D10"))
 (segment (start 98.35 69.5) (end 122.35 93.5) (width 0.2) (layer "B.Cu") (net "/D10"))
 (segment (start 92 69.5) (end 98.35 69.5) (width 0.2) (layer "B.Cu") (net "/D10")))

